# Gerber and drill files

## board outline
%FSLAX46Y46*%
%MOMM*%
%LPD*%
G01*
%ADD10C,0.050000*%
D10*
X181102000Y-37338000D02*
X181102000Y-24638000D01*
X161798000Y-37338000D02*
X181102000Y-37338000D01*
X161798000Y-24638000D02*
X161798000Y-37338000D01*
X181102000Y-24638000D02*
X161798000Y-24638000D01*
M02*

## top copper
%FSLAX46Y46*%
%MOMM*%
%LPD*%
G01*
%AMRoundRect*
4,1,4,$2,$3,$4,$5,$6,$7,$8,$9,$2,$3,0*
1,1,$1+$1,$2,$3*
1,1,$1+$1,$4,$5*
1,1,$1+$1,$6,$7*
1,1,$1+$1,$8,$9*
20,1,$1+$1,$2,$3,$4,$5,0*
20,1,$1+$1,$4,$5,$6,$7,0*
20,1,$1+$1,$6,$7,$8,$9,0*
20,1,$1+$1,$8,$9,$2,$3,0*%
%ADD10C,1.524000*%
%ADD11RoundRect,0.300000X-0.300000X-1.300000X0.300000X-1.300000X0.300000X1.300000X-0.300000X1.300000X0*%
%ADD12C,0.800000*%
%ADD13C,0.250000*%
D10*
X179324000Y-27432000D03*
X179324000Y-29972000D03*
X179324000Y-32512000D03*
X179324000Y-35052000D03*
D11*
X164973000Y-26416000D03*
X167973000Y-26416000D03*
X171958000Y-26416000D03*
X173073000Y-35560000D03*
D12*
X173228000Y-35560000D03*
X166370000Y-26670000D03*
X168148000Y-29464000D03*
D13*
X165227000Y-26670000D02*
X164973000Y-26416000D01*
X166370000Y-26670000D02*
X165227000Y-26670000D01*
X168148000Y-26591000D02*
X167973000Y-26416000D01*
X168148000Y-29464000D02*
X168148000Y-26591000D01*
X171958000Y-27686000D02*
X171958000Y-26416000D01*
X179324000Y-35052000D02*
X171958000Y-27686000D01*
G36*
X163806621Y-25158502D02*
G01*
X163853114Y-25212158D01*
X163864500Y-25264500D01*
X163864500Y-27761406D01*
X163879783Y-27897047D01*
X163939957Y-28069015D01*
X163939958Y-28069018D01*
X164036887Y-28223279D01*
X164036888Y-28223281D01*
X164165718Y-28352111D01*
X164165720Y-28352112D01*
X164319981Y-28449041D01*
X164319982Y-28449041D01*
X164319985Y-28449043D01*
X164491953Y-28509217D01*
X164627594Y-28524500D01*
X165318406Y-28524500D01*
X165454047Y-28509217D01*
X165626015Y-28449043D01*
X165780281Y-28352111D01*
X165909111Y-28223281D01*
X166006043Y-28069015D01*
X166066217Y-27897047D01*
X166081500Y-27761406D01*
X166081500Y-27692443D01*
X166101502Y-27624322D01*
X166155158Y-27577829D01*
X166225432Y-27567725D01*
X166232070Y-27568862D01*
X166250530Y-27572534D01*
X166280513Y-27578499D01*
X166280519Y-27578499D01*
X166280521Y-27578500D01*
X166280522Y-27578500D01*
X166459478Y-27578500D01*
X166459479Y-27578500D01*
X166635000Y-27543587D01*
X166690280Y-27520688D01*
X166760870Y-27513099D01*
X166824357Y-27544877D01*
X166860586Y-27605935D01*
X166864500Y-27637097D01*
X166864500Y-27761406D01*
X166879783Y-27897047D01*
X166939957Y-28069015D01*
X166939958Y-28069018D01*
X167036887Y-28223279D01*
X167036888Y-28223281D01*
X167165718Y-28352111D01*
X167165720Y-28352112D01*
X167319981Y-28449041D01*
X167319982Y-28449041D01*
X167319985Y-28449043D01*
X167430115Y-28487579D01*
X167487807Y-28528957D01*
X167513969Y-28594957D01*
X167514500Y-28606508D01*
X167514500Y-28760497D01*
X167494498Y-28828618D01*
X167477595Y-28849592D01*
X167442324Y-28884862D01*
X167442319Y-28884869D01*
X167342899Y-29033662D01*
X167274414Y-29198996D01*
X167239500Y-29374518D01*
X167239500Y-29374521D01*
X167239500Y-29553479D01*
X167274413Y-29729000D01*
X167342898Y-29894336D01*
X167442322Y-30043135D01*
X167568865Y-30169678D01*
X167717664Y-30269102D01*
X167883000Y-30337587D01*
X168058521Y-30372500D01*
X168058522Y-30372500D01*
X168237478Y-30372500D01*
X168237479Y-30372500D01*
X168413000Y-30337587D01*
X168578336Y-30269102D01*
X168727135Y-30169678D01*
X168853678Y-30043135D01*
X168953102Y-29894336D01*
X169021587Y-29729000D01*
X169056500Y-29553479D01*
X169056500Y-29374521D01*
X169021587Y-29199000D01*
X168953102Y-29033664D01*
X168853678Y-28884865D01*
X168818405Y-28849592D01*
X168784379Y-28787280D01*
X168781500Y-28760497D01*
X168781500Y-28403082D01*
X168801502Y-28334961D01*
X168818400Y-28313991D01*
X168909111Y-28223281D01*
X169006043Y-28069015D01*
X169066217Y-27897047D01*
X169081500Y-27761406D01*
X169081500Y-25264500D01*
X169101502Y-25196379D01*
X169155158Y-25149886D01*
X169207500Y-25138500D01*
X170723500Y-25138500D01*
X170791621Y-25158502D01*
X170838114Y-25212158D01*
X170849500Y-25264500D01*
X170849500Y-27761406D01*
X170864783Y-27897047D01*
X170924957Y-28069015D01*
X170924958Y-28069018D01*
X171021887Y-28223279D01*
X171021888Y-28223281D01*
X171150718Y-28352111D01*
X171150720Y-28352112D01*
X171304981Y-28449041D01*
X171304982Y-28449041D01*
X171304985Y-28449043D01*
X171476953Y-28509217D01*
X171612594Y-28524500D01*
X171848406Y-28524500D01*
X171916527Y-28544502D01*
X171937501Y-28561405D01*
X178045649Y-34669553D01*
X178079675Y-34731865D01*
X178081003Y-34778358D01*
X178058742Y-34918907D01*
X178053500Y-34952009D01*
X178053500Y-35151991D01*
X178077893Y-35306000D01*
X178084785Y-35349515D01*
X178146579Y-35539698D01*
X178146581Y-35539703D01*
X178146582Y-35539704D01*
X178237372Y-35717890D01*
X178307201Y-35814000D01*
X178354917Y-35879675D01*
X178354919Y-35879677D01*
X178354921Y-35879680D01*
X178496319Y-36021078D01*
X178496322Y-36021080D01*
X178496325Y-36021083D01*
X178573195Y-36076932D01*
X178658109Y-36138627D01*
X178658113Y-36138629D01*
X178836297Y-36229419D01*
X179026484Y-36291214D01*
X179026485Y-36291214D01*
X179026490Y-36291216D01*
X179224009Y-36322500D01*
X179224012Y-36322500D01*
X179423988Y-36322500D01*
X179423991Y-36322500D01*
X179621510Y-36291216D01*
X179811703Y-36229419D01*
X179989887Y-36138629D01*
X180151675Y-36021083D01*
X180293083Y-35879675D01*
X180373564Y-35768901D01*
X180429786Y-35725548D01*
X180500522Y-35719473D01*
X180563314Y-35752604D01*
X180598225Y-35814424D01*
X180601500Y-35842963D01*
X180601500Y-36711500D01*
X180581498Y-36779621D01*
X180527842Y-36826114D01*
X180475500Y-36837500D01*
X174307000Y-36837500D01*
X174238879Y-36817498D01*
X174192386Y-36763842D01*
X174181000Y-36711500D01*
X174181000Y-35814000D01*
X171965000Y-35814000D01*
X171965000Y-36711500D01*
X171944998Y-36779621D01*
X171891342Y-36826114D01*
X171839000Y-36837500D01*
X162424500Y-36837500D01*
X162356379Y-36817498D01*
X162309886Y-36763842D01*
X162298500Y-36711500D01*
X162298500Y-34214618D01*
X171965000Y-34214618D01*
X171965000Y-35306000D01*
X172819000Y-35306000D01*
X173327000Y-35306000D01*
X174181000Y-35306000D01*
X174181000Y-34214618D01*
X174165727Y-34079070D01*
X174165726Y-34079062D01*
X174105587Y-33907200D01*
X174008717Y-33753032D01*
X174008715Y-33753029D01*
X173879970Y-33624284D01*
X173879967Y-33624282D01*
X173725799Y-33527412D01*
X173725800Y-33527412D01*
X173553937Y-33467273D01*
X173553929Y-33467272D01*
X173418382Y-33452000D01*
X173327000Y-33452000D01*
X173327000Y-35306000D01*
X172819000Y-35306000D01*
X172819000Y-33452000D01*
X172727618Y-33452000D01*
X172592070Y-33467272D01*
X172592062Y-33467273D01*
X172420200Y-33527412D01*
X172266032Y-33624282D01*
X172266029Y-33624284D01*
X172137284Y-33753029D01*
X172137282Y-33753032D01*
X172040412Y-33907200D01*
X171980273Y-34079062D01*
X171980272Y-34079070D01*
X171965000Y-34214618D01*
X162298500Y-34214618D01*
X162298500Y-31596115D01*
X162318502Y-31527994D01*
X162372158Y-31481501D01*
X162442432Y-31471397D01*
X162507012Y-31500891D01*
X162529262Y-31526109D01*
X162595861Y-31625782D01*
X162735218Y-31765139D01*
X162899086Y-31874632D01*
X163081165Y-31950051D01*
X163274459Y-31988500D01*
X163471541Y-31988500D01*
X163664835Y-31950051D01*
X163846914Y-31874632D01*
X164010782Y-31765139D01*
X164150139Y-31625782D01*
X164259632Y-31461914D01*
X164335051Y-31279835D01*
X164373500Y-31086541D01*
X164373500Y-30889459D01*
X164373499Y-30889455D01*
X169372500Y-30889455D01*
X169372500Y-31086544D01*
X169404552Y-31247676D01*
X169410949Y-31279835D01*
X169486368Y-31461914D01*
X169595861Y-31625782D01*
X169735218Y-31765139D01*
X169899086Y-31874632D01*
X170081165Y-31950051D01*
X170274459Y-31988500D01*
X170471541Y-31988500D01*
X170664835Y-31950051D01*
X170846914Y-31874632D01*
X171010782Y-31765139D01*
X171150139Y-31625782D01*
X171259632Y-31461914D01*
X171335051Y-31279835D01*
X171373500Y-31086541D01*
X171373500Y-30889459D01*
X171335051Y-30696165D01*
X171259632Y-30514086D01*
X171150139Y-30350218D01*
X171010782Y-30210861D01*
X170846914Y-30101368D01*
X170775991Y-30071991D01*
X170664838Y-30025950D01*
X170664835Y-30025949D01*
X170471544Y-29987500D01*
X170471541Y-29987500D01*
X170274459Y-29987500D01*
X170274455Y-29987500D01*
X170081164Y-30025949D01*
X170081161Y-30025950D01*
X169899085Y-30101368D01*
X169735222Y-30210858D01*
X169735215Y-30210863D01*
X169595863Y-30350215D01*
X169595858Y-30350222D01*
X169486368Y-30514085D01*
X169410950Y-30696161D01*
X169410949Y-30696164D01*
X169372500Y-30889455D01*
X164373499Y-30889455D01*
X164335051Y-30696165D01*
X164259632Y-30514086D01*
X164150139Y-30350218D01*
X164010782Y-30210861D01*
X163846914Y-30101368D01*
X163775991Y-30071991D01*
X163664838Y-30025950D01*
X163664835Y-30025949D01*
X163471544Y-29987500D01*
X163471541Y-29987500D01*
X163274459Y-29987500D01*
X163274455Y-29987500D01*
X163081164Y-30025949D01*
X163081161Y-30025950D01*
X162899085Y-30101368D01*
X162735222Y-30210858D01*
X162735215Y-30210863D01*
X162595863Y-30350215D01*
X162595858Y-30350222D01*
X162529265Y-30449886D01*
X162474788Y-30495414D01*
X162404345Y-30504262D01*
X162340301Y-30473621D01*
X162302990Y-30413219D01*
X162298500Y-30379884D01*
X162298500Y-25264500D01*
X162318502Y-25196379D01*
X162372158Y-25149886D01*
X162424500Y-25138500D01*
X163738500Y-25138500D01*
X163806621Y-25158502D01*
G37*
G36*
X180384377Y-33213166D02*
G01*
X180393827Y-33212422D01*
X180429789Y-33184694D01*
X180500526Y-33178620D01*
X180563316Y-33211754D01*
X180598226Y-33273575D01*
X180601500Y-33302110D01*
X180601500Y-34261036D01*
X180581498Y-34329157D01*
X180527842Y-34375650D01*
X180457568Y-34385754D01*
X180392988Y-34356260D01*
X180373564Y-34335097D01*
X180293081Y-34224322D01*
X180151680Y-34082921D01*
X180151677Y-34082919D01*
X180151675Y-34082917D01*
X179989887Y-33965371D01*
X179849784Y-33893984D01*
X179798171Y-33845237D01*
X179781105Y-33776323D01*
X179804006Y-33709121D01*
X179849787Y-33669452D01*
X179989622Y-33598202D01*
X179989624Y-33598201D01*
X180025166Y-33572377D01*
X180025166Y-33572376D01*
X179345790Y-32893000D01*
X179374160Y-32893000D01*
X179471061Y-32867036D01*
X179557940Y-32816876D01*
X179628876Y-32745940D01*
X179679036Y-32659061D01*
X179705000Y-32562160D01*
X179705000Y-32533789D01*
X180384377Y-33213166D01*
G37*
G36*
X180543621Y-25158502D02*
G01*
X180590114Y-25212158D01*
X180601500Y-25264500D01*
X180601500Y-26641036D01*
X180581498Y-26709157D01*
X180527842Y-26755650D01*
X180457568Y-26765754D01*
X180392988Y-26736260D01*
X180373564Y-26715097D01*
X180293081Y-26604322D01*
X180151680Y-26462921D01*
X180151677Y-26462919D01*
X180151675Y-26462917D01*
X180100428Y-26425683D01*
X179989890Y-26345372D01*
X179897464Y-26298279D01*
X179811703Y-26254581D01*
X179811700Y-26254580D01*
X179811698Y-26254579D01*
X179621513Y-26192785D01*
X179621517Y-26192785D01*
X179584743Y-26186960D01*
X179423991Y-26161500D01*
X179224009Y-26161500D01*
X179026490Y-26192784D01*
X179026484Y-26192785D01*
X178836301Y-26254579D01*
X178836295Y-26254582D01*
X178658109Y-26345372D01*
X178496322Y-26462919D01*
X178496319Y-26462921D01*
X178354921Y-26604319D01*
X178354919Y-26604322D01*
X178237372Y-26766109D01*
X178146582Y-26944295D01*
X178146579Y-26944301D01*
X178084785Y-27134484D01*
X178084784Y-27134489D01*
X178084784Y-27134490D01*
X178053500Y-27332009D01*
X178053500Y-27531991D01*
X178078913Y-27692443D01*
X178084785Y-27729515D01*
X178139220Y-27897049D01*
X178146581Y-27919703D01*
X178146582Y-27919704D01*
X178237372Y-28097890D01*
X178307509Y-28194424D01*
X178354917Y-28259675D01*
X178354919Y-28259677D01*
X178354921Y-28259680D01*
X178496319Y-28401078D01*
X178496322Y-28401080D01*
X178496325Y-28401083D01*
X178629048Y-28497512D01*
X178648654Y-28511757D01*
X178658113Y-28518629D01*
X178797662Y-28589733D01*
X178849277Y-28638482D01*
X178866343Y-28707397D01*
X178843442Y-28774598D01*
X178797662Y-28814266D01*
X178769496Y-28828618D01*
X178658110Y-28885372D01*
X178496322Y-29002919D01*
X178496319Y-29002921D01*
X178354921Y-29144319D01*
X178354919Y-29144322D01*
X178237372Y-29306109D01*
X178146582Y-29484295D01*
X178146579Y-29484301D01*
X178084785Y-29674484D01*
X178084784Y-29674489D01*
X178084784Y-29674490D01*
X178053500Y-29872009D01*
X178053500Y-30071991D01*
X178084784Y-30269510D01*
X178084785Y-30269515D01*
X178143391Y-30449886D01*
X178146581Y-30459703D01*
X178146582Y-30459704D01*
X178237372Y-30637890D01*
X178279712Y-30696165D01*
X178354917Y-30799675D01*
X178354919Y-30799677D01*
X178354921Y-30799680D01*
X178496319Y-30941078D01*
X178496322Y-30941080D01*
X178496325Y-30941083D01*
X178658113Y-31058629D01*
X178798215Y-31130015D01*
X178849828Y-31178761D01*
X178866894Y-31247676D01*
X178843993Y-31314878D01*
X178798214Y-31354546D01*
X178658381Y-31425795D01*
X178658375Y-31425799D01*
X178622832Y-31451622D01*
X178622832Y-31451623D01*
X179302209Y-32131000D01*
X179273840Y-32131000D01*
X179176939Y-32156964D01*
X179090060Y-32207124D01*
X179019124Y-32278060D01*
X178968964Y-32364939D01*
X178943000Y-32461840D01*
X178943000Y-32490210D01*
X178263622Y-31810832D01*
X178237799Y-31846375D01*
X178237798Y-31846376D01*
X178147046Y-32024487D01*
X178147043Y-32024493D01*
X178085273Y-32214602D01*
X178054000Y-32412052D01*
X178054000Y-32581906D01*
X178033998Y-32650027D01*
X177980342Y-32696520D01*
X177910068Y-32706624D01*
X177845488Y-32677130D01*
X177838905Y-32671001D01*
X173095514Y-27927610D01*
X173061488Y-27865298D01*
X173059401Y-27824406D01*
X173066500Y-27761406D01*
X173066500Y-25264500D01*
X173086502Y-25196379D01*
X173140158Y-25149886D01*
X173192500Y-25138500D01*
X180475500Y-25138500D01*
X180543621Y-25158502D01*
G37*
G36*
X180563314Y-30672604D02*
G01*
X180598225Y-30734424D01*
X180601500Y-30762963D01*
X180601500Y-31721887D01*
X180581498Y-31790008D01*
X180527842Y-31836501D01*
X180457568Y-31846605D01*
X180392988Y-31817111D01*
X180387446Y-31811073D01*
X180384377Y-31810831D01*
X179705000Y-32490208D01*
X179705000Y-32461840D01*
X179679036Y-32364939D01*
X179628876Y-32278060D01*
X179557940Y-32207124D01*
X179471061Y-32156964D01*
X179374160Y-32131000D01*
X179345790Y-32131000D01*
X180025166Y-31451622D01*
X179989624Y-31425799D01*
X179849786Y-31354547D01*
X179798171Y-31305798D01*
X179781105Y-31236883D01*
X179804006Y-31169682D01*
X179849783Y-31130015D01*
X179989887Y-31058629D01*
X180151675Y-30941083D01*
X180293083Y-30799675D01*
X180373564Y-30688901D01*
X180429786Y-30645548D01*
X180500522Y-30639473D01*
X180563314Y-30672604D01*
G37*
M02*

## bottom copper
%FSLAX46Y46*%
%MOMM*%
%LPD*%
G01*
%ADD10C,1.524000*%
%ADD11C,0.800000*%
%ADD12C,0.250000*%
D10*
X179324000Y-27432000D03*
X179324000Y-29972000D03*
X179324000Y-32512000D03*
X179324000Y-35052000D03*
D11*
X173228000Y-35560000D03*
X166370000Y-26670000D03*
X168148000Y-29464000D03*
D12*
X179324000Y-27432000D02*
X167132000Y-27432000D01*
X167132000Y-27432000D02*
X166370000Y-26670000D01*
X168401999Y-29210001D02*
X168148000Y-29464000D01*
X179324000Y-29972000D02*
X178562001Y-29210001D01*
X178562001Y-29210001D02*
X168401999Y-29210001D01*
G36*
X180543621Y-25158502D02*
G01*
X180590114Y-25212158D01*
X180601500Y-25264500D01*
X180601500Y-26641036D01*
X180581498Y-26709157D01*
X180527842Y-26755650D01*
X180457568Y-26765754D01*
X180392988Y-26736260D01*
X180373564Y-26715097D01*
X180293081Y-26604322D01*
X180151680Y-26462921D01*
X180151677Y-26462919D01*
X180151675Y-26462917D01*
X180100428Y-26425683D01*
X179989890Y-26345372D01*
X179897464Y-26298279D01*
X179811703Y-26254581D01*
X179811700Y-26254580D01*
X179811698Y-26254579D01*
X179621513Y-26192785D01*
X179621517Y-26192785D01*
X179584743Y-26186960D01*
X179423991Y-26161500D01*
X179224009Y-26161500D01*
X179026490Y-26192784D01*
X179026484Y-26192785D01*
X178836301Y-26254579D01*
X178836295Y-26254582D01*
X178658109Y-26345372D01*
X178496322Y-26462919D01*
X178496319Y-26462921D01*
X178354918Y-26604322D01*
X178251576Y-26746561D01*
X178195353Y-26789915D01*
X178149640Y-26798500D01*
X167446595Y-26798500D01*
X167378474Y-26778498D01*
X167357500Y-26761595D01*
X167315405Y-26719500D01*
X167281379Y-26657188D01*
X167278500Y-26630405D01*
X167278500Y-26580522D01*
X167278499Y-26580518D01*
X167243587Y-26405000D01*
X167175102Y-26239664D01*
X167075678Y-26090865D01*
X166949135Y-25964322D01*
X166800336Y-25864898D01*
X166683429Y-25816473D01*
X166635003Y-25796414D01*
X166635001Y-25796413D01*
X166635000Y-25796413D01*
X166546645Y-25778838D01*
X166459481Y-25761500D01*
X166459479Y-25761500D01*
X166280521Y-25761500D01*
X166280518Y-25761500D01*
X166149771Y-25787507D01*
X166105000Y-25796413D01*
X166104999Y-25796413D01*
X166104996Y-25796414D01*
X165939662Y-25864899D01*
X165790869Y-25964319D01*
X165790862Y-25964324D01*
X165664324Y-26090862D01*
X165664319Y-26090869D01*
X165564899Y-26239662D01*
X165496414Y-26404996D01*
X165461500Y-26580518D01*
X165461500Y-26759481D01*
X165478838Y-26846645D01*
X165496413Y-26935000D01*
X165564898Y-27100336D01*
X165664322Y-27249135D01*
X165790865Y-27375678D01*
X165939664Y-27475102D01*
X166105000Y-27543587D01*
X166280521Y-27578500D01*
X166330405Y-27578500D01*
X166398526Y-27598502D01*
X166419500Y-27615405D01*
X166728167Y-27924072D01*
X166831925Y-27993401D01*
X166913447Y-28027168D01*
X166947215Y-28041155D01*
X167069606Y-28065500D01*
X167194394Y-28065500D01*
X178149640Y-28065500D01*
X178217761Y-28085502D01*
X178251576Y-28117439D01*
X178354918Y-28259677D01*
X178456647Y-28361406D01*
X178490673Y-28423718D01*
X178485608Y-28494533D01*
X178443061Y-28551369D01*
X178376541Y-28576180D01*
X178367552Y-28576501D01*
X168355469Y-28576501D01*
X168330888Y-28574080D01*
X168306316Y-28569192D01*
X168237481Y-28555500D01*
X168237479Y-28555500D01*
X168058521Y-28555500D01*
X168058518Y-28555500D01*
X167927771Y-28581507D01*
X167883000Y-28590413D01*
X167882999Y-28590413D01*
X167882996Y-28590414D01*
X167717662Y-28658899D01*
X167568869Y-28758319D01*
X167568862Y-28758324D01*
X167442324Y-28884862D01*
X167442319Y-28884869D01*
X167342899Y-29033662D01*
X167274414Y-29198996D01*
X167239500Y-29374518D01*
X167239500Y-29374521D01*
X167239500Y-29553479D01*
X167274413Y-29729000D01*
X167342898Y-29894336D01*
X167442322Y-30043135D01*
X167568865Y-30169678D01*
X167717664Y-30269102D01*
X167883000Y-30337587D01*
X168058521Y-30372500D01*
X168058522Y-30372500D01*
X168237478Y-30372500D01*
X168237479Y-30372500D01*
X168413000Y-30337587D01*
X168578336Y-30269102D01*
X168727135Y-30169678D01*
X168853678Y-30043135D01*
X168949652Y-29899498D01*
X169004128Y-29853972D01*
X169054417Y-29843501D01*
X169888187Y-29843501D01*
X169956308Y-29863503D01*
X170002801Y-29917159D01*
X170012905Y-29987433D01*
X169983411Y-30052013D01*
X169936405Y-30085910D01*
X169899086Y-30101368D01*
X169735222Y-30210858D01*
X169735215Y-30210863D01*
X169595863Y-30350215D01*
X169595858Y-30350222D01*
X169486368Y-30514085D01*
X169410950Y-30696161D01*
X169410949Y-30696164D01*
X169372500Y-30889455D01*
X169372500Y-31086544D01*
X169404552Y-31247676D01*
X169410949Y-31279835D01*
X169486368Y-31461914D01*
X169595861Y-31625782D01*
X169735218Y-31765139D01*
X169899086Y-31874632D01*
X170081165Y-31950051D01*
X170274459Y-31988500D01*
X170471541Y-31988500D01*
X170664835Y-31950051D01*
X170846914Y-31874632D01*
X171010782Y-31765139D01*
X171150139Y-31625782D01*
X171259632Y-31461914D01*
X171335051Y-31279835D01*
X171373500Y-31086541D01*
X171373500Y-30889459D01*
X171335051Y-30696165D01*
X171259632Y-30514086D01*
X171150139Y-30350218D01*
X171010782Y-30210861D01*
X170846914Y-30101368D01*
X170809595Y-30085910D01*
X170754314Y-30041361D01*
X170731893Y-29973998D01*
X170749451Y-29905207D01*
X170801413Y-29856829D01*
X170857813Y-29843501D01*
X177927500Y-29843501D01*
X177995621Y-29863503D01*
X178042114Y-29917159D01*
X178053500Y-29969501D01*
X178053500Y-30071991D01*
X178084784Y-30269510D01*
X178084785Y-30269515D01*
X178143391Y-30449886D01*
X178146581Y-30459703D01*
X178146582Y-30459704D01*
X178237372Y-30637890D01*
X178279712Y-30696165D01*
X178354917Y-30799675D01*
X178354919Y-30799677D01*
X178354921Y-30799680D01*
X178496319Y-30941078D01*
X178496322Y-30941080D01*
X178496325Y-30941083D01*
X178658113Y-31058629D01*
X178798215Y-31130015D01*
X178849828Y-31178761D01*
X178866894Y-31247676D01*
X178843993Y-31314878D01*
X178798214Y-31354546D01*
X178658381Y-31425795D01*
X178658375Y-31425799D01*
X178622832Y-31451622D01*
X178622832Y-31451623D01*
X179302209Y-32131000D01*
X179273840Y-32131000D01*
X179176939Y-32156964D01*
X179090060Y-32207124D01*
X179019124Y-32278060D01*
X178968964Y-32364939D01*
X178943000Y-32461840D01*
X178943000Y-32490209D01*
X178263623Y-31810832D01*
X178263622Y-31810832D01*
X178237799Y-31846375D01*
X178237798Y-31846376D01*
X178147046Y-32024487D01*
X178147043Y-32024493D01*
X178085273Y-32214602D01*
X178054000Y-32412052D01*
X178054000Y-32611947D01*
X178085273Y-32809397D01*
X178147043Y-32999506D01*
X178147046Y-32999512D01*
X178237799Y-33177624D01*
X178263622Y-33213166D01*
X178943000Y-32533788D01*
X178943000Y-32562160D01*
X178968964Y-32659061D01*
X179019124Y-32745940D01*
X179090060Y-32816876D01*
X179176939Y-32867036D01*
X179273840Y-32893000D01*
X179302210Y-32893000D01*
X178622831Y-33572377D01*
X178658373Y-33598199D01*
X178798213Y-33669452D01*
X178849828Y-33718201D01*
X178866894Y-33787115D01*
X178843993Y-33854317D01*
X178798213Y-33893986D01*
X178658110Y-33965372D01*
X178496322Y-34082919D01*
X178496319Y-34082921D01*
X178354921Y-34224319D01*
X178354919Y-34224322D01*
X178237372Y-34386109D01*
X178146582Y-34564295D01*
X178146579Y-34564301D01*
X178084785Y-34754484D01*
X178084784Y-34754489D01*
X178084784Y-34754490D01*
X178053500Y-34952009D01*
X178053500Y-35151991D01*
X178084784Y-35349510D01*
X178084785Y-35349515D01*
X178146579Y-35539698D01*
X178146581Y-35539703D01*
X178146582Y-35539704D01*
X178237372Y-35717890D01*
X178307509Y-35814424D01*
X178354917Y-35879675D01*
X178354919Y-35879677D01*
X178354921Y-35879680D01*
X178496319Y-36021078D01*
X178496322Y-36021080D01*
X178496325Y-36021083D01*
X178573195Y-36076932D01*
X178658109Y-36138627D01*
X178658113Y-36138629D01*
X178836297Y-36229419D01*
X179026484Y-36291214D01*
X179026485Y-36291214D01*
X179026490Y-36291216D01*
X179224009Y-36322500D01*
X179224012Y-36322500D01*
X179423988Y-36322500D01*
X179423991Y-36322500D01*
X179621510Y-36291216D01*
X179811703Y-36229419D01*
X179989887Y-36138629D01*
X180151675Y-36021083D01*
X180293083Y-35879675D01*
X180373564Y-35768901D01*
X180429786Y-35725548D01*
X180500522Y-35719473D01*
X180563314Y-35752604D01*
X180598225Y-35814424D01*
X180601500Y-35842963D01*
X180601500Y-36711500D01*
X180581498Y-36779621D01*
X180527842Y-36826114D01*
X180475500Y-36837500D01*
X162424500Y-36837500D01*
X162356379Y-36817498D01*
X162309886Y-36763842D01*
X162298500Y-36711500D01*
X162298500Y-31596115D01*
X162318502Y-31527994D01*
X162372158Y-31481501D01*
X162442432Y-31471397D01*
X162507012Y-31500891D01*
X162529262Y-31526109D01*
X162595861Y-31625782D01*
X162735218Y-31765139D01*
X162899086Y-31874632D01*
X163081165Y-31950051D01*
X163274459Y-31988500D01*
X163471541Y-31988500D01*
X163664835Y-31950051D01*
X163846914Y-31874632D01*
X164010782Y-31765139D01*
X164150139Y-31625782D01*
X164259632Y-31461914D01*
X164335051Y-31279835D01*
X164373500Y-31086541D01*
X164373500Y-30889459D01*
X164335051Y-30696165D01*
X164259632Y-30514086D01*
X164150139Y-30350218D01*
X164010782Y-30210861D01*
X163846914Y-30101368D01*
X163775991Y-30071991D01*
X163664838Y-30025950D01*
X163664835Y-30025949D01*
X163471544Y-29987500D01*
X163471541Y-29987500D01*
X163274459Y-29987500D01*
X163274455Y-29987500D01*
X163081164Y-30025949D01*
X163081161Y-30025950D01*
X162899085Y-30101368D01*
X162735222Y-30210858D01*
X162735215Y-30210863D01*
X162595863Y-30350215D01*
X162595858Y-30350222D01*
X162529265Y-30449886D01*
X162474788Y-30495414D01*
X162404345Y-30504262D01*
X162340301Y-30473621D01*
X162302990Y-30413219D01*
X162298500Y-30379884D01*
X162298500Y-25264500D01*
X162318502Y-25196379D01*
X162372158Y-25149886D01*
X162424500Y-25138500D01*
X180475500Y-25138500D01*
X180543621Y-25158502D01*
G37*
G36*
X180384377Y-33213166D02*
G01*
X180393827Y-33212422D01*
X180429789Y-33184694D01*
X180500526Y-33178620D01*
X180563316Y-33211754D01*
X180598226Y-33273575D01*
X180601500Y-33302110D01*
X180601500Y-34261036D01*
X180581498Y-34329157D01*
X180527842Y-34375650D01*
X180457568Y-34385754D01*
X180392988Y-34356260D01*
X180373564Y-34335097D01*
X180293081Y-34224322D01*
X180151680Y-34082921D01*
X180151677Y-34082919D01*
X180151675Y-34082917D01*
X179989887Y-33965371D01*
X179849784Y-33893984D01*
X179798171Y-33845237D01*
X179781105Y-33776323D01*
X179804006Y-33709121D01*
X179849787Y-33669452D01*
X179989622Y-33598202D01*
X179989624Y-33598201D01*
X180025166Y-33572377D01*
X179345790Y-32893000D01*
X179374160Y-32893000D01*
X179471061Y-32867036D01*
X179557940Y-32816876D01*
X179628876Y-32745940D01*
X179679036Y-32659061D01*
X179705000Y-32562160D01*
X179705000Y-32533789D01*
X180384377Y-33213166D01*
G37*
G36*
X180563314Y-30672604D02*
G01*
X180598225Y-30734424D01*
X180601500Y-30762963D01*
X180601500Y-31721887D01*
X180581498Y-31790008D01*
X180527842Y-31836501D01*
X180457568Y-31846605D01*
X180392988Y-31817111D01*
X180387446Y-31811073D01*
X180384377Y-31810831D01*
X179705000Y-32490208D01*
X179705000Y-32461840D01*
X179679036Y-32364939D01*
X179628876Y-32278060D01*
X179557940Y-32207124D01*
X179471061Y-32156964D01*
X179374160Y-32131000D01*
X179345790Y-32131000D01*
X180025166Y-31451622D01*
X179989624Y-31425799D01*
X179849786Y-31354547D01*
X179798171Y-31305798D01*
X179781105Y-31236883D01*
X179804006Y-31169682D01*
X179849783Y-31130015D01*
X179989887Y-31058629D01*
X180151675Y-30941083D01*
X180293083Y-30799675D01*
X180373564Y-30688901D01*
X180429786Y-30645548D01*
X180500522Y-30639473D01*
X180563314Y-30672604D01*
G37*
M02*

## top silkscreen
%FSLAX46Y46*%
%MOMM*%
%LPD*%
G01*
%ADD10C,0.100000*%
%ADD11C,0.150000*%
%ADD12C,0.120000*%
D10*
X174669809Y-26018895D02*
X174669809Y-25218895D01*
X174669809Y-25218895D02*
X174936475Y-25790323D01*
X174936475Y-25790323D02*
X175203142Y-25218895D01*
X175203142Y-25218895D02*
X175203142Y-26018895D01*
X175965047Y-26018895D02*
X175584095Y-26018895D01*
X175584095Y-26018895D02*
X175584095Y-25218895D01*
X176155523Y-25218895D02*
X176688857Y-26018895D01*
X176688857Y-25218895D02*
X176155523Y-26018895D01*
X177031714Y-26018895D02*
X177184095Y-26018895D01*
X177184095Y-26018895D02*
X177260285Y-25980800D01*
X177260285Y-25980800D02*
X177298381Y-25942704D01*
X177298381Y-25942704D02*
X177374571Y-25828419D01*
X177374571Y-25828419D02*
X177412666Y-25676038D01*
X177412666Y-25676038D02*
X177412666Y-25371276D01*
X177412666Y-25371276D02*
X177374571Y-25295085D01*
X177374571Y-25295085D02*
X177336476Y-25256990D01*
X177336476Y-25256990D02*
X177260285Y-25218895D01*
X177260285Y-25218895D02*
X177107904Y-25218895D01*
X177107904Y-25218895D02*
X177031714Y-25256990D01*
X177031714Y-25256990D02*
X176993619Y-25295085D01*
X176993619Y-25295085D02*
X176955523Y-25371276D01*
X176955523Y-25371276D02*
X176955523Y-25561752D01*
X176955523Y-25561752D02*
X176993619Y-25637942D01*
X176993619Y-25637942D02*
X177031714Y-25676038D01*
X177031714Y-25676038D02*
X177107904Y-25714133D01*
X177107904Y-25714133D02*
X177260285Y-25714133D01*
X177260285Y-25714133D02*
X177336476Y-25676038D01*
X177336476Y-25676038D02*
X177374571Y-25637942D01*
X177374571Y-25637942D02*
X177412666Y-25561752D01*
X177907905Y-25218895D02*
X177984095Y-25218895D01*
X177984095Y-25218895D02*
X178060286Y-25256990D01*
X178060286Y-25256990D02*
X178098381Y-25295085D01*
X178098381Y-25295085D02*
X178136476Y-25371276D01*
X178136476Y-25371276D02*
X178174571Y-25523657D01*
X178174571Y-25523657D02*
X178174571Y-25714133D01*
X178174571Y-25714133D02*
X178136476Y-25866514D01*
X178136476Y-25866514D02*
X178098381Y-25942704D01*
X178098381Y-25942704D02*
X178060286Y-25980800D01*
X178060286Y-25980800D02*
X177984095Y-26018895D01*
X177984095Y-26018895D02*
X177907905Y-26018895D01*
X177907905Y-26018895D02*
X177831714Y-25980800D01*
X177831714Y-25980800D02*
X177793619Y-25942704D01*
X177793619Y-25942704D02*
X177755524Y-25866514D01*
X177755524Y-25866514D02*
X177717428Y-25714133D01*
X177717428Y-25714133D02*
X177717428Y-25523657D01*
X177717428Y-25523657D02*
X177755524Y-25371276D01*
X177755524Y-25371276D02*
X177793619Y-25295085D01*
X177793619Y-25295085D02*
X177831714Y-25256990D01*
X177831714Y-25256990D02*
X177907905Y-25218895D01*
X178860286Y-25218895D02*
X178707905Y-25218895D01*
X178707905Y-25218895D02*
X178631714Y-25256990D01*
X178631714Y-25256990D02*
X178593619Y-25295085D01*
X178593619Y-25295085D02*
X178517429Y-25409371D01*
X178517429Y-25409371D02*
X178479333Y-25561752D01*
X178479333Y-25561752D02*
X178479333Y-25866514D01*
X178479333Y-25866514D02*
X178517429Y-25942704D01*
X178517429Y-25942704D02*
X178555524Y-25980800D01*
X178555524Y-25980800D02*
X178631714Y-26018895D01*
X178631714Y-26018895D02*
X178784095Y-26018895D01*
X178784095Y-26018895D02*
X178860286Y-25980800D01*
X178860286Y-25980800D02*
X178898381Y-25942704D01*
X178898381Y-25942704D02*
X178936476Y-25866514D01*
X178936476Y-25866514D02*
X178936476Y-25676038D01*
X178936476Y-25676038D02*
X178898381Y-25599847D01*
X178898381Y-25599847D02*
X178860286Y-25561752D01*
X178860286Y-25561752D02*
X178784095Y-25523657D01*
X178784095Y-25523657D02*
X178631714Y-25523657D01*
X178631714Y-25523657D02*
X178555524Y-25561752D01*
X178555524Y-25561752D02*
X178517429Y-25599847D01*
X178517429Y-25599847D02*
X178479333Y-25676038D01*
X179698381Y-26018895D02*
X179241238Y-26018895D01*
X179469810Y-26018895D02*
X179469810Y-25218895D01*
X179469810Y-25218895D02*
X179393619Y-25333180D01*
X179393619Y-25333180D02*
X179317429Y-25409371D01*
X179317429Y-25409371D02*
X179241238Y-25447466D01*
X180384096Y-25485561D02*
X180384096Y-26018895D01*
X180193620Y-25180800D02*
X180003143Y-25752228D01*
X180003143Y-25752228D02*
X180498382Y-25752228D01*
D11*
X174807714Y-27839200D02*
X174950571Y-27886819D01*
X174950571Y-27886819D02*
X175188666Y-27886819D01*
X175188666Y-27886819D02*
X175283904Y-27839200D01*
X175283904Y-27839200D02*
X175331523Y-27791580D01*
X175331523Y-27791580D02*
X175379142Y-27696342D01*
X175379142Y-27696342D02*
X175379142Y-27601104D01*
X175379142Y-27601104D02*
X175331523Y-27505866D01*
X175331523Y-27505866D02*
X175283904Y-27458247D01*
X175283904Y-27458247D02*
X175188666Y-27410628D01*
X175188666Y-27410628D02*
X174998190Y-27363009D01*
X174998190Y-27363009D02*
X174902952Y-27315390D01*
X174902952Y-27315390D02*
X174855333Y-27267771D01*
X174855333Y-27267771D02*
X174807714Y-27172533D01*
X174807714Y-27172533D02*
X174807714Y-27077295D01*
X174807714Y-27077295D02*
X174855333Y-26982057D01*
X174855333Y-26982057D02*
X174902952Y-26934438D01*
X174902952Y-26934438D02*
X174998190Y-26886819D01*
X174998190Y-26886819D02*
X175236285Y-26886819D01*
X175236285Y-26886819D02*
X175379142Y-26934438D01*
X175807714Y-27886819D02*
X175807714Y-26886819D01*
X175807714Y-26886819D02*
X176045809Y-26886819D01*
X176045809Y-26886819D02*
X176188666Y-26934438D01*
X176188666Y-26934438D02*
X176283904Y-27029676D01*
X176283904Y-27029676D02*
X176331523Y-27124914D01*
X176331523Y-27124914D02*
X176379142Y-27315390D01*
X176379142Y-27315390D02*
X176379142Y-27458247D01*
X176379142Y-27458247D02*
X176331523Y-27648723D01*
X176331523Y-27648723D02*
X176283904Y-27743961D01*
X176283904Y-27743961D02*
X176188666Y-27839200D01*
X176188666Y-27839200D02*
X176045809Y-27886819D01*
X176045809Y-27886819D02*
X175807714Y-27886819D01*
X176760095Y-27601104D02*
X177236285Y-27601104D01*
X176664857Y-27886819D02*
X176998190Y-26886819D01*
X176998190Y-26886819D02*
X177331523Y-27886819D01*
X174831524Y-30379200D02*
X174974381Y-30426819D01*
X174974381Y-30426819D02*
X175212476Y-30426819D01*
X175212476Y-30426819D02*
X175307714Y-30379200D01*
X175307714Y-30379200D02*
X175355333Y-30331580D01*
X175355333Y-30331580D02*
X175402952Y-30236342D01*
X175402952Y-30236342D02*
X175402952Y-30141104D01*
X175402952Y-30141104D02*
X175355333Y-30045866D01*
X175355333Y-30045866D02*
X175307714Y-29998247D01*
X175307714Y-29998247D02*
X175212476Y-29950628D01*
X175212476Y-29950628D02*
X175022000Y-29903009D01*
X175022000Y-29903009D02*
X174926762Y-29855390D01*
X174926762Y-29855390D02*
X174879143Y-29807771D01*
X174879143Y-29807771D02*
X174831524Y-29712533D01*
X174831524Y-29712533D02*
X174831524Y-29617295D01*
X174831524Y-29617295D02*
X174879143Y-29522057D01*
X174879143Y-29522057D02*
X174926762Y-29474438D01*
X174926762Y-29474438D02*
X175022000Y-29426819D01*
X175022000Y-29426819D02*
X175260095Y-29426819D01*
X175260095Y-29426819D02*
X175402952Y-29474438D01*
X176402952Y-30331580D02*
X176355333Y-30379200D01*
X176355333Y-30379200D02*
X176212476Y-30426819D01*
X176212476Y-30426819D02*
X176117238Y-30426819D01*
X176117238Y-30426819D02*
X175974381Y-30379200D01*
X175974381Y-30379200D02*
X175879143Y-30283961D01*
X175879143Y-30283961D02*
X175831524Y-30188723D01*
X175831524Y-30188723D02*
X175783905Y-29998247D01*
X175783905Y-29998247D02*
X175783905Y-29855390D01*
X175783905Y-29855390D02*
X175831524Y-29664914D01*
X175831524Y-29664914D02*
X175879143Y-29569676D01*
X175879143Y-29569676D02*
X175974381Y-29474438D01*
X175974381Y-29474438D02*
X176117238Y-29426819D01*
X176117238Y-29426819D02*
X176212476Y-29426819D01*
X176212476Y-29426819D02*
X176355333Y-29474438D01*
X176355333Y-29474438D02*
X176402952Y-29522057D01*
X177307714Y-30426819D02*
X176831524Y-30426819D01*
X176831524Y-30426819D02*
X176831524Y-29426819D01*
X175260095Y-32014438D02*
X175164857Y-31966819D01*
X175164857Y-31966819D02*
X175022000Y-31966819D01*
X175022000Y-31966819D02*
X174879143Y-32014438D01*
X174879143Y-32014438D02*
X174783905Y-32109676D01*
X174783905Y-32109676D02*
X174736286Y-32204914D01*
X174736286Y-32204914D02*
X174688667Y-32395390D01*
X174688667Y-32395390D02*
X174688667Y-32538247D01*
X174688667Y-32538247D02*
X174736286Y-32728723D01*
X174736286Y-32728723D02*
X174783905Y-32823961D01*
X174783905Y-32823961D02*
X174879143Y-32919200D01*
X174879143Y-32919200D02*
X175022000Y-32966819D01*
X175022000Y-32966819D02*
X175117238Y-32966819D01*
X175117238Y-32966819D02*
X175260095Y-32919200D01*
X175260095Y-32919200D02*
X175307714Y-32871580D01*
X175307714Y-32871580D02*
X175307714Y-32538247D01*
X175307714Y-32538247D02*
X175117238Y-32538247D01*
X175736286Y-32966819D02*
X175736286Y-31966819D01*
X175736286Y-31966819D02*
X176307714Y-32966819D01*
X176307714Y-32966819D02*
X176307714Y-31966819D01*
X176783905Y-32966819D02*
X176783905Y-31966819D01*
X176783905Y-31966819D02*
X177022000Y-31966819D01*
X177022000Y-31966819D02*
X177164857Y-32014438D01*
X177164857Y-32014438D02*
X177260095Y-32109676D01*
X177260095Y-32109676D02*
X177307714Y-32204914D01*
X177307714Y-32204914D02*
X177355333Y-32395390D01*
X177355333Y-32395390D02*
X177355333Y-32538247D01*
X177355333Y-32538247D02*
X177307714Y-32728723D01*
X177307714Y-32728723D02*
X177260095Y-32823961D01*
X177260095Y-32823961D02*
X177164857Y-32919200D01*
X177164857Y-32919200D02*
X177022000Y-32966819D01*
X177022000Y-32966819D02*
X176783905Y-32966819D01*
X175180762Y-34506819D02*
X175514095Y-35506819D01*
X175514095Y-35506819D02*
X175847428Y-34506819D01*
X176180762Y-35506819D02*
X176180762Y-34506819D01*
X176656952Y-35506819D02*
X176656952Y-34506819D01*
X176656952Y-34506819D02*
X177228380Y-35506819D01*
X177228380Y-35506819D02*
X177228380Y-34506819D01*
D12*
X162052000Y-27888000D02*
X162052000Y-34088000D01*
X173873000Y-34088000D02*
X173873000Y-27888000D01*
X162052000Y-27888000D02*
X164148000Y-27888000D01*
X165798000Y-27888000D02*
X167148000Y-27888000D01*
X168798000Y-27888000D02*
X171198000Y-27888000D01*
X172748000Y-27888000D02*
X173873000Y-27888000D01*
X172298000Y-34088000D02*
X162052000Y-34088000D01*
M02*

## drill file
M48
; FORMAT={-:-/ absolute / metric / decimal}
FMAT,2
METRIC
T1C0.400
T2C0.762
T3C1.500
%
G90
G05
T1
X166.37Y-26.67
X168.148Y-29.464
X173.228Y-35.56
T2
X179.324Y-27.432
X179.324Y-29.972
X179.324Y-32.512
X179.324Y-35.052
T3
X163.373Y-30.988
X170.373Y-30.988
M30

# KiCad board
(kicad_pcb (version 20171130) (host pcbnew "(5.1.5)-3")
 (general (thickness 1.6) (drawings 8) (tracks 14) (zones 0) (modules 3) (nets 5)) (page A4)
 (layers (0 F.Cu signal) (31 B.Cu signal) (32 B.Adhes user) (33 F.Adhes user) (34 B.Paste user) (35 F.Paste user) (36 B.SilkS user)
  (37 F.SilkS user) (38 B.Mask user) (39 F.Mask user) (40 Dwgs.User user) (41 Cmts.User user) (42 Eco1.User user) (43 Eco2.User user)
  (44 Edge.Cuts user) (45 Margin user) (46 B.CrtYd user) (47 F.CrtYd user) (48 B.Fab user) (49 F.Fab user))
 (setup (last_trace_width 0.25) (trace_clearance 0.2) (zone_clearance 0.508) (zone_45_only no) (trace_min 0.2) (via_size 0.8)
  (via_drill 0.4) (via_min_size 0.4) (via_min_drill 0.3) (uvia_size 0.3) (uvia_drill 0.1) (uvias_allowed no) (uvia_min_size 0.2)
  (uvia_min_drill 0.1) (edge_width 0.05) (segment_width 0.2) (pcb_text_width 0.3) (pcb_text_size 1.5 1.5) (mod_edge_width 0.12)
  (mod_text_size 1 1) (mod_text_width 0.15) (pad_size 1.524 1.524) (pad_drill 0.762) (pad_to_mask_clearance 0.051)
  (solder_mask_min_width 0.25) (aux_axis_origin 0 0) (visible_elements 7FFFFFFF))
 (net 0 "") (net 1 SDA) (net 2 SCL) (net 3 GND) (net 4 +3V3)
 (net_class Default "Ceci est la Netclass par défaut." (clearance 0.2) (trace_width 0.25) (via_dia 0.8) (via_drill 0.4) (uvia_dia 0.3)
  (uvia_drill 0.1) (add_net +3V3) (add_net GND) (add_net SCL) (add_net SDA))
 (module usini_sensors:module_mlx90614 (layer F.Cu) (at 179.324 27.432 180)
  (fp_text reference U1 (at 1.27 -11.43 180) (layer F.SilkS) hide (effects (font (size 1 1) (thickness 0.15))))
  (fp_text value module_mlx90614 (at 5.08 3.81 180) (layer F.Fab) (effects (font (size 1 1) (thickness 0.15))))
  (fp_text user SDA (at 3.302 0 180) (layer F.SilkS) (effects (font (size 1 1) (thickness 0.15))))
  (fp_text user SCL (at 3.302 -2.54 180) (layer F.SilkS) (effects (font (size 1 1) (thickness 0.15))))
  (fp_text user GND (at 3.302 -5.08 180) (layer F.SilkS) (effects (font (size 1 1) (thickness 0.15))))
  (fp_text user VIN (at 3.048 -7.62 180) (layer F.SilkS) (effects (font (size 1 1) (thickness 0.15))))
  (pad 4 thru_hole circle (at 0 0 180) (size 1.524 1.524) (drill 0.762) (layers *.Cu *.Mask) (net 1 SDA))
  (pad 3 thru_hole circle (at 0 -2.54 180) (size 1.524 1.524) (drill 0.762) (layers *.Cu *.Mask) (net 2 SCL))
  (pad 2 thru_hole circle (at 0 -5.08 180) (size 1.524 1.524) (drill 0.762) (layers *.Cu *.Mask) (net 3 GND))
  (pad 1 thru_hole circle (at 0 -7.62 180) (size 1.524 1.524) (drill 0.762) (layers *.Cu *.Mask) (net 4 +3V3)))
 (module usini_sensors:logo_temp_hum (layer B.Cu) (at 168.91 27.432 180)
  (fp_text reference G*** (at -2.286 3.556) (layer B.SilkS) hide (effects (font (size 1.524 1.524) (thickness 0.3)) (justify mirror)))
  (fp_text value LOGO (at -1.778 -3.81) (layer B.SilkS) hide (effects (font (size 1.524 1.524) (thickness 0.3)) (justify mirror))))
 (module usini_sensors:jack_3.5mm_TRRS (layer F.Cu) (at 168.148 30.988)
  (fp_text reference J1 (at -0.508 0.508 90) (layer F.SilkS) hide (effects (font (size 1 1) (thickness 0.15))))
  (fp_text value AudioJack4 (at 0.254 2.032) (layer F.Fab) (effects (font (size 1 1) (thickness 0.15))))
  (fp_line (start -6.096 -3.1) (end -6.096 3.1) (layer F.SilkS) (width 0.12))
  (fp_line (start 5.725 3.1) (end 5.725 -3.1) (layer F.SilkS) (width 0.12))
  (fp_line (start -6.096 -3.1) (end -4 -3.1) (layer F.SilkS) (width 0.12))
  (fp_line (start -2.35 -3.1) (end -1 -3.1) (layer F.SilkS) (width 0.12))
  (fp_line (start 0.65 -3.1) (end 3.05 -3.1) (layer F.SilkS) (width 0.12))
  (fp_line (start 4.6 -3.1) (end 5.725 -3.1) (layer F.SilkS) (width 0.12))
  (fp_line (start 4.15 3.1) (end -6.096 3.1) (layer F.SilkS) (width 0.12))
  (pad "" np_thru_hole circle (at 2.225 0) (size 1.5 1.5) (drill 1.5) (layers *.Cu *.Mask))
  (pad "" np_thru_hole circle (at -4.775 0) (size 1.5 1.5) (drill 1.5) (layers *.Cu *.Mask))
  (pad R2 smd roundrect (at -3.175 -4.572) (size 1.2 3.2) (layers F.Cu F.Paste F.Mask) (roundrect_rratio 0.25) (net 1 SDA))
  (pad R1 smd roundrect (at -0.175 -4.572) (size 1.2 3.2) (layers F.Cu F.Paste F.Mask) (roundrect_rratio 0.25) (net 2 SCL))
  (pad T smd roundrect (at 3.81 -4.572) (size 1.2 3.2) (layers F.Cu F.Paste F.Mask) (roundrect_rratio 0.25) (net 4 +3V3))
  (pad S smd roundrect (at 4.925 4.572) (size 1.2 3.2) (layers F.Cu F.Paste F.Mask) (roundrect_rratio 0.25) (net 3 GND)))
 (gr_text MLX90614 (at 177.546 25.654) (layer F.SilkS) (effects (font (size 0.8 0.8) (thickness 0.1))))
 (gr_line (start 181.102 37.338) (end 181.102 24.638) (layer Edge.Cuts) (width 0.05))
 (gr_line (start 161.798 37.338) (end 181.102 37.338) (layer Edge.Cuts) (width 0.05))
 (gr_line (start 161.798 24.638) (end 161.798 37.338) (layer Edge.Cuts) (width 0.05))
 (gr_line (start 181.102 24.638) (end 161.798 24.638) (layer Edge.Cuts) (width 0.05))
 (via (at 173.228 35.56) (size 0.8) (drill 0.4) (layers F.Cu B.Cu) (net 3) (status 30))
 (via (at 166.37 26.67) (size 0.8) (drill 0.4) (layers F.Cu B.Cu) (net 1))
 (segment (start 179.324 27.432) (end 167.132 27.432) (width 0.25) (layer B.Cu) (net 1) (status 10))
 (segment (start 167.132 27.432) (end 166.37 26.67) (width 0.25) (layer B.Cu) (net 1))
 (segment (start 165.227 26.67) (end 164.973 26.416) (width 0.25) (layer F.Cu) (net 1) (status 30))
 (segment (start 166.37 26.67) (end 165.227 26.67) (width 0.25) (layer F.Cu) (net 1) (status 20))
 (via (at 168.148 29.464) (size 0.8) (drill 0.4) (layers F.Cu B.Cu) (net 2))
 (segment (start 168.401999 29.210001) (end 168.148 29.464) (width 0.25) (layer B.Cu) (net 2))
 (segment (start 179.324 29.972) (end 178.562001 29.210001) (width 0.25) (layer B.Cu) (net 2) (status 10))
 (segment (start 178.562001 29.210001) (end 168.401999 29.210001) (width 0.25) (layer B.Cu) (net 2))
 (segment (start 168.148 26.591) (end 167.973 26.416) (width 0.25) (layer F.Cu) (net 2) (status 30))
 (segment (start 168.148 29.464) (end 168.148 26.591) (width 0.25) (layer F.Cu) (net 2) (status 20))
 (segment (start 171.958 27.686) (end 171.958 26.416) (width 0.25) (layer F.Cu) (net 4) (status 30))
 (segment (start 179.324 35.052) (end 171.958 27.686) (width 0.25) (layer F.Cu) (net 4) (status 30))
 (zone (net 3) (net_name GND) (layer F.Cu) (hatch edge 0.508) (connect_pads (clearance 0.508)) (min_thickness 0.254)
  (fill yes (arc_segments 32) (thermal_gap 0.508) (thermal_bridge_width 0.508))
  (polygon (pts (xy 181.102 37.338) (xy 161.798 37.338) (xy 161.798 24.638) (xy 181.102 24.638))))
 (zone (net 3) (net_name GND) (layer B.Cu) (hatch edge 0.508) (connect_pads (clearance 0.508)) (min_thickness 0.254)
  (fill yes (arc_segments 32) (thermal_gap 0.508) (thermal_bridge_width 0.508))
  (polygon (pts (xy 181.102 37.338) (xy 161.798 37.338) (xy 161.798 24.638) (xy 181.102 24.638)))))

